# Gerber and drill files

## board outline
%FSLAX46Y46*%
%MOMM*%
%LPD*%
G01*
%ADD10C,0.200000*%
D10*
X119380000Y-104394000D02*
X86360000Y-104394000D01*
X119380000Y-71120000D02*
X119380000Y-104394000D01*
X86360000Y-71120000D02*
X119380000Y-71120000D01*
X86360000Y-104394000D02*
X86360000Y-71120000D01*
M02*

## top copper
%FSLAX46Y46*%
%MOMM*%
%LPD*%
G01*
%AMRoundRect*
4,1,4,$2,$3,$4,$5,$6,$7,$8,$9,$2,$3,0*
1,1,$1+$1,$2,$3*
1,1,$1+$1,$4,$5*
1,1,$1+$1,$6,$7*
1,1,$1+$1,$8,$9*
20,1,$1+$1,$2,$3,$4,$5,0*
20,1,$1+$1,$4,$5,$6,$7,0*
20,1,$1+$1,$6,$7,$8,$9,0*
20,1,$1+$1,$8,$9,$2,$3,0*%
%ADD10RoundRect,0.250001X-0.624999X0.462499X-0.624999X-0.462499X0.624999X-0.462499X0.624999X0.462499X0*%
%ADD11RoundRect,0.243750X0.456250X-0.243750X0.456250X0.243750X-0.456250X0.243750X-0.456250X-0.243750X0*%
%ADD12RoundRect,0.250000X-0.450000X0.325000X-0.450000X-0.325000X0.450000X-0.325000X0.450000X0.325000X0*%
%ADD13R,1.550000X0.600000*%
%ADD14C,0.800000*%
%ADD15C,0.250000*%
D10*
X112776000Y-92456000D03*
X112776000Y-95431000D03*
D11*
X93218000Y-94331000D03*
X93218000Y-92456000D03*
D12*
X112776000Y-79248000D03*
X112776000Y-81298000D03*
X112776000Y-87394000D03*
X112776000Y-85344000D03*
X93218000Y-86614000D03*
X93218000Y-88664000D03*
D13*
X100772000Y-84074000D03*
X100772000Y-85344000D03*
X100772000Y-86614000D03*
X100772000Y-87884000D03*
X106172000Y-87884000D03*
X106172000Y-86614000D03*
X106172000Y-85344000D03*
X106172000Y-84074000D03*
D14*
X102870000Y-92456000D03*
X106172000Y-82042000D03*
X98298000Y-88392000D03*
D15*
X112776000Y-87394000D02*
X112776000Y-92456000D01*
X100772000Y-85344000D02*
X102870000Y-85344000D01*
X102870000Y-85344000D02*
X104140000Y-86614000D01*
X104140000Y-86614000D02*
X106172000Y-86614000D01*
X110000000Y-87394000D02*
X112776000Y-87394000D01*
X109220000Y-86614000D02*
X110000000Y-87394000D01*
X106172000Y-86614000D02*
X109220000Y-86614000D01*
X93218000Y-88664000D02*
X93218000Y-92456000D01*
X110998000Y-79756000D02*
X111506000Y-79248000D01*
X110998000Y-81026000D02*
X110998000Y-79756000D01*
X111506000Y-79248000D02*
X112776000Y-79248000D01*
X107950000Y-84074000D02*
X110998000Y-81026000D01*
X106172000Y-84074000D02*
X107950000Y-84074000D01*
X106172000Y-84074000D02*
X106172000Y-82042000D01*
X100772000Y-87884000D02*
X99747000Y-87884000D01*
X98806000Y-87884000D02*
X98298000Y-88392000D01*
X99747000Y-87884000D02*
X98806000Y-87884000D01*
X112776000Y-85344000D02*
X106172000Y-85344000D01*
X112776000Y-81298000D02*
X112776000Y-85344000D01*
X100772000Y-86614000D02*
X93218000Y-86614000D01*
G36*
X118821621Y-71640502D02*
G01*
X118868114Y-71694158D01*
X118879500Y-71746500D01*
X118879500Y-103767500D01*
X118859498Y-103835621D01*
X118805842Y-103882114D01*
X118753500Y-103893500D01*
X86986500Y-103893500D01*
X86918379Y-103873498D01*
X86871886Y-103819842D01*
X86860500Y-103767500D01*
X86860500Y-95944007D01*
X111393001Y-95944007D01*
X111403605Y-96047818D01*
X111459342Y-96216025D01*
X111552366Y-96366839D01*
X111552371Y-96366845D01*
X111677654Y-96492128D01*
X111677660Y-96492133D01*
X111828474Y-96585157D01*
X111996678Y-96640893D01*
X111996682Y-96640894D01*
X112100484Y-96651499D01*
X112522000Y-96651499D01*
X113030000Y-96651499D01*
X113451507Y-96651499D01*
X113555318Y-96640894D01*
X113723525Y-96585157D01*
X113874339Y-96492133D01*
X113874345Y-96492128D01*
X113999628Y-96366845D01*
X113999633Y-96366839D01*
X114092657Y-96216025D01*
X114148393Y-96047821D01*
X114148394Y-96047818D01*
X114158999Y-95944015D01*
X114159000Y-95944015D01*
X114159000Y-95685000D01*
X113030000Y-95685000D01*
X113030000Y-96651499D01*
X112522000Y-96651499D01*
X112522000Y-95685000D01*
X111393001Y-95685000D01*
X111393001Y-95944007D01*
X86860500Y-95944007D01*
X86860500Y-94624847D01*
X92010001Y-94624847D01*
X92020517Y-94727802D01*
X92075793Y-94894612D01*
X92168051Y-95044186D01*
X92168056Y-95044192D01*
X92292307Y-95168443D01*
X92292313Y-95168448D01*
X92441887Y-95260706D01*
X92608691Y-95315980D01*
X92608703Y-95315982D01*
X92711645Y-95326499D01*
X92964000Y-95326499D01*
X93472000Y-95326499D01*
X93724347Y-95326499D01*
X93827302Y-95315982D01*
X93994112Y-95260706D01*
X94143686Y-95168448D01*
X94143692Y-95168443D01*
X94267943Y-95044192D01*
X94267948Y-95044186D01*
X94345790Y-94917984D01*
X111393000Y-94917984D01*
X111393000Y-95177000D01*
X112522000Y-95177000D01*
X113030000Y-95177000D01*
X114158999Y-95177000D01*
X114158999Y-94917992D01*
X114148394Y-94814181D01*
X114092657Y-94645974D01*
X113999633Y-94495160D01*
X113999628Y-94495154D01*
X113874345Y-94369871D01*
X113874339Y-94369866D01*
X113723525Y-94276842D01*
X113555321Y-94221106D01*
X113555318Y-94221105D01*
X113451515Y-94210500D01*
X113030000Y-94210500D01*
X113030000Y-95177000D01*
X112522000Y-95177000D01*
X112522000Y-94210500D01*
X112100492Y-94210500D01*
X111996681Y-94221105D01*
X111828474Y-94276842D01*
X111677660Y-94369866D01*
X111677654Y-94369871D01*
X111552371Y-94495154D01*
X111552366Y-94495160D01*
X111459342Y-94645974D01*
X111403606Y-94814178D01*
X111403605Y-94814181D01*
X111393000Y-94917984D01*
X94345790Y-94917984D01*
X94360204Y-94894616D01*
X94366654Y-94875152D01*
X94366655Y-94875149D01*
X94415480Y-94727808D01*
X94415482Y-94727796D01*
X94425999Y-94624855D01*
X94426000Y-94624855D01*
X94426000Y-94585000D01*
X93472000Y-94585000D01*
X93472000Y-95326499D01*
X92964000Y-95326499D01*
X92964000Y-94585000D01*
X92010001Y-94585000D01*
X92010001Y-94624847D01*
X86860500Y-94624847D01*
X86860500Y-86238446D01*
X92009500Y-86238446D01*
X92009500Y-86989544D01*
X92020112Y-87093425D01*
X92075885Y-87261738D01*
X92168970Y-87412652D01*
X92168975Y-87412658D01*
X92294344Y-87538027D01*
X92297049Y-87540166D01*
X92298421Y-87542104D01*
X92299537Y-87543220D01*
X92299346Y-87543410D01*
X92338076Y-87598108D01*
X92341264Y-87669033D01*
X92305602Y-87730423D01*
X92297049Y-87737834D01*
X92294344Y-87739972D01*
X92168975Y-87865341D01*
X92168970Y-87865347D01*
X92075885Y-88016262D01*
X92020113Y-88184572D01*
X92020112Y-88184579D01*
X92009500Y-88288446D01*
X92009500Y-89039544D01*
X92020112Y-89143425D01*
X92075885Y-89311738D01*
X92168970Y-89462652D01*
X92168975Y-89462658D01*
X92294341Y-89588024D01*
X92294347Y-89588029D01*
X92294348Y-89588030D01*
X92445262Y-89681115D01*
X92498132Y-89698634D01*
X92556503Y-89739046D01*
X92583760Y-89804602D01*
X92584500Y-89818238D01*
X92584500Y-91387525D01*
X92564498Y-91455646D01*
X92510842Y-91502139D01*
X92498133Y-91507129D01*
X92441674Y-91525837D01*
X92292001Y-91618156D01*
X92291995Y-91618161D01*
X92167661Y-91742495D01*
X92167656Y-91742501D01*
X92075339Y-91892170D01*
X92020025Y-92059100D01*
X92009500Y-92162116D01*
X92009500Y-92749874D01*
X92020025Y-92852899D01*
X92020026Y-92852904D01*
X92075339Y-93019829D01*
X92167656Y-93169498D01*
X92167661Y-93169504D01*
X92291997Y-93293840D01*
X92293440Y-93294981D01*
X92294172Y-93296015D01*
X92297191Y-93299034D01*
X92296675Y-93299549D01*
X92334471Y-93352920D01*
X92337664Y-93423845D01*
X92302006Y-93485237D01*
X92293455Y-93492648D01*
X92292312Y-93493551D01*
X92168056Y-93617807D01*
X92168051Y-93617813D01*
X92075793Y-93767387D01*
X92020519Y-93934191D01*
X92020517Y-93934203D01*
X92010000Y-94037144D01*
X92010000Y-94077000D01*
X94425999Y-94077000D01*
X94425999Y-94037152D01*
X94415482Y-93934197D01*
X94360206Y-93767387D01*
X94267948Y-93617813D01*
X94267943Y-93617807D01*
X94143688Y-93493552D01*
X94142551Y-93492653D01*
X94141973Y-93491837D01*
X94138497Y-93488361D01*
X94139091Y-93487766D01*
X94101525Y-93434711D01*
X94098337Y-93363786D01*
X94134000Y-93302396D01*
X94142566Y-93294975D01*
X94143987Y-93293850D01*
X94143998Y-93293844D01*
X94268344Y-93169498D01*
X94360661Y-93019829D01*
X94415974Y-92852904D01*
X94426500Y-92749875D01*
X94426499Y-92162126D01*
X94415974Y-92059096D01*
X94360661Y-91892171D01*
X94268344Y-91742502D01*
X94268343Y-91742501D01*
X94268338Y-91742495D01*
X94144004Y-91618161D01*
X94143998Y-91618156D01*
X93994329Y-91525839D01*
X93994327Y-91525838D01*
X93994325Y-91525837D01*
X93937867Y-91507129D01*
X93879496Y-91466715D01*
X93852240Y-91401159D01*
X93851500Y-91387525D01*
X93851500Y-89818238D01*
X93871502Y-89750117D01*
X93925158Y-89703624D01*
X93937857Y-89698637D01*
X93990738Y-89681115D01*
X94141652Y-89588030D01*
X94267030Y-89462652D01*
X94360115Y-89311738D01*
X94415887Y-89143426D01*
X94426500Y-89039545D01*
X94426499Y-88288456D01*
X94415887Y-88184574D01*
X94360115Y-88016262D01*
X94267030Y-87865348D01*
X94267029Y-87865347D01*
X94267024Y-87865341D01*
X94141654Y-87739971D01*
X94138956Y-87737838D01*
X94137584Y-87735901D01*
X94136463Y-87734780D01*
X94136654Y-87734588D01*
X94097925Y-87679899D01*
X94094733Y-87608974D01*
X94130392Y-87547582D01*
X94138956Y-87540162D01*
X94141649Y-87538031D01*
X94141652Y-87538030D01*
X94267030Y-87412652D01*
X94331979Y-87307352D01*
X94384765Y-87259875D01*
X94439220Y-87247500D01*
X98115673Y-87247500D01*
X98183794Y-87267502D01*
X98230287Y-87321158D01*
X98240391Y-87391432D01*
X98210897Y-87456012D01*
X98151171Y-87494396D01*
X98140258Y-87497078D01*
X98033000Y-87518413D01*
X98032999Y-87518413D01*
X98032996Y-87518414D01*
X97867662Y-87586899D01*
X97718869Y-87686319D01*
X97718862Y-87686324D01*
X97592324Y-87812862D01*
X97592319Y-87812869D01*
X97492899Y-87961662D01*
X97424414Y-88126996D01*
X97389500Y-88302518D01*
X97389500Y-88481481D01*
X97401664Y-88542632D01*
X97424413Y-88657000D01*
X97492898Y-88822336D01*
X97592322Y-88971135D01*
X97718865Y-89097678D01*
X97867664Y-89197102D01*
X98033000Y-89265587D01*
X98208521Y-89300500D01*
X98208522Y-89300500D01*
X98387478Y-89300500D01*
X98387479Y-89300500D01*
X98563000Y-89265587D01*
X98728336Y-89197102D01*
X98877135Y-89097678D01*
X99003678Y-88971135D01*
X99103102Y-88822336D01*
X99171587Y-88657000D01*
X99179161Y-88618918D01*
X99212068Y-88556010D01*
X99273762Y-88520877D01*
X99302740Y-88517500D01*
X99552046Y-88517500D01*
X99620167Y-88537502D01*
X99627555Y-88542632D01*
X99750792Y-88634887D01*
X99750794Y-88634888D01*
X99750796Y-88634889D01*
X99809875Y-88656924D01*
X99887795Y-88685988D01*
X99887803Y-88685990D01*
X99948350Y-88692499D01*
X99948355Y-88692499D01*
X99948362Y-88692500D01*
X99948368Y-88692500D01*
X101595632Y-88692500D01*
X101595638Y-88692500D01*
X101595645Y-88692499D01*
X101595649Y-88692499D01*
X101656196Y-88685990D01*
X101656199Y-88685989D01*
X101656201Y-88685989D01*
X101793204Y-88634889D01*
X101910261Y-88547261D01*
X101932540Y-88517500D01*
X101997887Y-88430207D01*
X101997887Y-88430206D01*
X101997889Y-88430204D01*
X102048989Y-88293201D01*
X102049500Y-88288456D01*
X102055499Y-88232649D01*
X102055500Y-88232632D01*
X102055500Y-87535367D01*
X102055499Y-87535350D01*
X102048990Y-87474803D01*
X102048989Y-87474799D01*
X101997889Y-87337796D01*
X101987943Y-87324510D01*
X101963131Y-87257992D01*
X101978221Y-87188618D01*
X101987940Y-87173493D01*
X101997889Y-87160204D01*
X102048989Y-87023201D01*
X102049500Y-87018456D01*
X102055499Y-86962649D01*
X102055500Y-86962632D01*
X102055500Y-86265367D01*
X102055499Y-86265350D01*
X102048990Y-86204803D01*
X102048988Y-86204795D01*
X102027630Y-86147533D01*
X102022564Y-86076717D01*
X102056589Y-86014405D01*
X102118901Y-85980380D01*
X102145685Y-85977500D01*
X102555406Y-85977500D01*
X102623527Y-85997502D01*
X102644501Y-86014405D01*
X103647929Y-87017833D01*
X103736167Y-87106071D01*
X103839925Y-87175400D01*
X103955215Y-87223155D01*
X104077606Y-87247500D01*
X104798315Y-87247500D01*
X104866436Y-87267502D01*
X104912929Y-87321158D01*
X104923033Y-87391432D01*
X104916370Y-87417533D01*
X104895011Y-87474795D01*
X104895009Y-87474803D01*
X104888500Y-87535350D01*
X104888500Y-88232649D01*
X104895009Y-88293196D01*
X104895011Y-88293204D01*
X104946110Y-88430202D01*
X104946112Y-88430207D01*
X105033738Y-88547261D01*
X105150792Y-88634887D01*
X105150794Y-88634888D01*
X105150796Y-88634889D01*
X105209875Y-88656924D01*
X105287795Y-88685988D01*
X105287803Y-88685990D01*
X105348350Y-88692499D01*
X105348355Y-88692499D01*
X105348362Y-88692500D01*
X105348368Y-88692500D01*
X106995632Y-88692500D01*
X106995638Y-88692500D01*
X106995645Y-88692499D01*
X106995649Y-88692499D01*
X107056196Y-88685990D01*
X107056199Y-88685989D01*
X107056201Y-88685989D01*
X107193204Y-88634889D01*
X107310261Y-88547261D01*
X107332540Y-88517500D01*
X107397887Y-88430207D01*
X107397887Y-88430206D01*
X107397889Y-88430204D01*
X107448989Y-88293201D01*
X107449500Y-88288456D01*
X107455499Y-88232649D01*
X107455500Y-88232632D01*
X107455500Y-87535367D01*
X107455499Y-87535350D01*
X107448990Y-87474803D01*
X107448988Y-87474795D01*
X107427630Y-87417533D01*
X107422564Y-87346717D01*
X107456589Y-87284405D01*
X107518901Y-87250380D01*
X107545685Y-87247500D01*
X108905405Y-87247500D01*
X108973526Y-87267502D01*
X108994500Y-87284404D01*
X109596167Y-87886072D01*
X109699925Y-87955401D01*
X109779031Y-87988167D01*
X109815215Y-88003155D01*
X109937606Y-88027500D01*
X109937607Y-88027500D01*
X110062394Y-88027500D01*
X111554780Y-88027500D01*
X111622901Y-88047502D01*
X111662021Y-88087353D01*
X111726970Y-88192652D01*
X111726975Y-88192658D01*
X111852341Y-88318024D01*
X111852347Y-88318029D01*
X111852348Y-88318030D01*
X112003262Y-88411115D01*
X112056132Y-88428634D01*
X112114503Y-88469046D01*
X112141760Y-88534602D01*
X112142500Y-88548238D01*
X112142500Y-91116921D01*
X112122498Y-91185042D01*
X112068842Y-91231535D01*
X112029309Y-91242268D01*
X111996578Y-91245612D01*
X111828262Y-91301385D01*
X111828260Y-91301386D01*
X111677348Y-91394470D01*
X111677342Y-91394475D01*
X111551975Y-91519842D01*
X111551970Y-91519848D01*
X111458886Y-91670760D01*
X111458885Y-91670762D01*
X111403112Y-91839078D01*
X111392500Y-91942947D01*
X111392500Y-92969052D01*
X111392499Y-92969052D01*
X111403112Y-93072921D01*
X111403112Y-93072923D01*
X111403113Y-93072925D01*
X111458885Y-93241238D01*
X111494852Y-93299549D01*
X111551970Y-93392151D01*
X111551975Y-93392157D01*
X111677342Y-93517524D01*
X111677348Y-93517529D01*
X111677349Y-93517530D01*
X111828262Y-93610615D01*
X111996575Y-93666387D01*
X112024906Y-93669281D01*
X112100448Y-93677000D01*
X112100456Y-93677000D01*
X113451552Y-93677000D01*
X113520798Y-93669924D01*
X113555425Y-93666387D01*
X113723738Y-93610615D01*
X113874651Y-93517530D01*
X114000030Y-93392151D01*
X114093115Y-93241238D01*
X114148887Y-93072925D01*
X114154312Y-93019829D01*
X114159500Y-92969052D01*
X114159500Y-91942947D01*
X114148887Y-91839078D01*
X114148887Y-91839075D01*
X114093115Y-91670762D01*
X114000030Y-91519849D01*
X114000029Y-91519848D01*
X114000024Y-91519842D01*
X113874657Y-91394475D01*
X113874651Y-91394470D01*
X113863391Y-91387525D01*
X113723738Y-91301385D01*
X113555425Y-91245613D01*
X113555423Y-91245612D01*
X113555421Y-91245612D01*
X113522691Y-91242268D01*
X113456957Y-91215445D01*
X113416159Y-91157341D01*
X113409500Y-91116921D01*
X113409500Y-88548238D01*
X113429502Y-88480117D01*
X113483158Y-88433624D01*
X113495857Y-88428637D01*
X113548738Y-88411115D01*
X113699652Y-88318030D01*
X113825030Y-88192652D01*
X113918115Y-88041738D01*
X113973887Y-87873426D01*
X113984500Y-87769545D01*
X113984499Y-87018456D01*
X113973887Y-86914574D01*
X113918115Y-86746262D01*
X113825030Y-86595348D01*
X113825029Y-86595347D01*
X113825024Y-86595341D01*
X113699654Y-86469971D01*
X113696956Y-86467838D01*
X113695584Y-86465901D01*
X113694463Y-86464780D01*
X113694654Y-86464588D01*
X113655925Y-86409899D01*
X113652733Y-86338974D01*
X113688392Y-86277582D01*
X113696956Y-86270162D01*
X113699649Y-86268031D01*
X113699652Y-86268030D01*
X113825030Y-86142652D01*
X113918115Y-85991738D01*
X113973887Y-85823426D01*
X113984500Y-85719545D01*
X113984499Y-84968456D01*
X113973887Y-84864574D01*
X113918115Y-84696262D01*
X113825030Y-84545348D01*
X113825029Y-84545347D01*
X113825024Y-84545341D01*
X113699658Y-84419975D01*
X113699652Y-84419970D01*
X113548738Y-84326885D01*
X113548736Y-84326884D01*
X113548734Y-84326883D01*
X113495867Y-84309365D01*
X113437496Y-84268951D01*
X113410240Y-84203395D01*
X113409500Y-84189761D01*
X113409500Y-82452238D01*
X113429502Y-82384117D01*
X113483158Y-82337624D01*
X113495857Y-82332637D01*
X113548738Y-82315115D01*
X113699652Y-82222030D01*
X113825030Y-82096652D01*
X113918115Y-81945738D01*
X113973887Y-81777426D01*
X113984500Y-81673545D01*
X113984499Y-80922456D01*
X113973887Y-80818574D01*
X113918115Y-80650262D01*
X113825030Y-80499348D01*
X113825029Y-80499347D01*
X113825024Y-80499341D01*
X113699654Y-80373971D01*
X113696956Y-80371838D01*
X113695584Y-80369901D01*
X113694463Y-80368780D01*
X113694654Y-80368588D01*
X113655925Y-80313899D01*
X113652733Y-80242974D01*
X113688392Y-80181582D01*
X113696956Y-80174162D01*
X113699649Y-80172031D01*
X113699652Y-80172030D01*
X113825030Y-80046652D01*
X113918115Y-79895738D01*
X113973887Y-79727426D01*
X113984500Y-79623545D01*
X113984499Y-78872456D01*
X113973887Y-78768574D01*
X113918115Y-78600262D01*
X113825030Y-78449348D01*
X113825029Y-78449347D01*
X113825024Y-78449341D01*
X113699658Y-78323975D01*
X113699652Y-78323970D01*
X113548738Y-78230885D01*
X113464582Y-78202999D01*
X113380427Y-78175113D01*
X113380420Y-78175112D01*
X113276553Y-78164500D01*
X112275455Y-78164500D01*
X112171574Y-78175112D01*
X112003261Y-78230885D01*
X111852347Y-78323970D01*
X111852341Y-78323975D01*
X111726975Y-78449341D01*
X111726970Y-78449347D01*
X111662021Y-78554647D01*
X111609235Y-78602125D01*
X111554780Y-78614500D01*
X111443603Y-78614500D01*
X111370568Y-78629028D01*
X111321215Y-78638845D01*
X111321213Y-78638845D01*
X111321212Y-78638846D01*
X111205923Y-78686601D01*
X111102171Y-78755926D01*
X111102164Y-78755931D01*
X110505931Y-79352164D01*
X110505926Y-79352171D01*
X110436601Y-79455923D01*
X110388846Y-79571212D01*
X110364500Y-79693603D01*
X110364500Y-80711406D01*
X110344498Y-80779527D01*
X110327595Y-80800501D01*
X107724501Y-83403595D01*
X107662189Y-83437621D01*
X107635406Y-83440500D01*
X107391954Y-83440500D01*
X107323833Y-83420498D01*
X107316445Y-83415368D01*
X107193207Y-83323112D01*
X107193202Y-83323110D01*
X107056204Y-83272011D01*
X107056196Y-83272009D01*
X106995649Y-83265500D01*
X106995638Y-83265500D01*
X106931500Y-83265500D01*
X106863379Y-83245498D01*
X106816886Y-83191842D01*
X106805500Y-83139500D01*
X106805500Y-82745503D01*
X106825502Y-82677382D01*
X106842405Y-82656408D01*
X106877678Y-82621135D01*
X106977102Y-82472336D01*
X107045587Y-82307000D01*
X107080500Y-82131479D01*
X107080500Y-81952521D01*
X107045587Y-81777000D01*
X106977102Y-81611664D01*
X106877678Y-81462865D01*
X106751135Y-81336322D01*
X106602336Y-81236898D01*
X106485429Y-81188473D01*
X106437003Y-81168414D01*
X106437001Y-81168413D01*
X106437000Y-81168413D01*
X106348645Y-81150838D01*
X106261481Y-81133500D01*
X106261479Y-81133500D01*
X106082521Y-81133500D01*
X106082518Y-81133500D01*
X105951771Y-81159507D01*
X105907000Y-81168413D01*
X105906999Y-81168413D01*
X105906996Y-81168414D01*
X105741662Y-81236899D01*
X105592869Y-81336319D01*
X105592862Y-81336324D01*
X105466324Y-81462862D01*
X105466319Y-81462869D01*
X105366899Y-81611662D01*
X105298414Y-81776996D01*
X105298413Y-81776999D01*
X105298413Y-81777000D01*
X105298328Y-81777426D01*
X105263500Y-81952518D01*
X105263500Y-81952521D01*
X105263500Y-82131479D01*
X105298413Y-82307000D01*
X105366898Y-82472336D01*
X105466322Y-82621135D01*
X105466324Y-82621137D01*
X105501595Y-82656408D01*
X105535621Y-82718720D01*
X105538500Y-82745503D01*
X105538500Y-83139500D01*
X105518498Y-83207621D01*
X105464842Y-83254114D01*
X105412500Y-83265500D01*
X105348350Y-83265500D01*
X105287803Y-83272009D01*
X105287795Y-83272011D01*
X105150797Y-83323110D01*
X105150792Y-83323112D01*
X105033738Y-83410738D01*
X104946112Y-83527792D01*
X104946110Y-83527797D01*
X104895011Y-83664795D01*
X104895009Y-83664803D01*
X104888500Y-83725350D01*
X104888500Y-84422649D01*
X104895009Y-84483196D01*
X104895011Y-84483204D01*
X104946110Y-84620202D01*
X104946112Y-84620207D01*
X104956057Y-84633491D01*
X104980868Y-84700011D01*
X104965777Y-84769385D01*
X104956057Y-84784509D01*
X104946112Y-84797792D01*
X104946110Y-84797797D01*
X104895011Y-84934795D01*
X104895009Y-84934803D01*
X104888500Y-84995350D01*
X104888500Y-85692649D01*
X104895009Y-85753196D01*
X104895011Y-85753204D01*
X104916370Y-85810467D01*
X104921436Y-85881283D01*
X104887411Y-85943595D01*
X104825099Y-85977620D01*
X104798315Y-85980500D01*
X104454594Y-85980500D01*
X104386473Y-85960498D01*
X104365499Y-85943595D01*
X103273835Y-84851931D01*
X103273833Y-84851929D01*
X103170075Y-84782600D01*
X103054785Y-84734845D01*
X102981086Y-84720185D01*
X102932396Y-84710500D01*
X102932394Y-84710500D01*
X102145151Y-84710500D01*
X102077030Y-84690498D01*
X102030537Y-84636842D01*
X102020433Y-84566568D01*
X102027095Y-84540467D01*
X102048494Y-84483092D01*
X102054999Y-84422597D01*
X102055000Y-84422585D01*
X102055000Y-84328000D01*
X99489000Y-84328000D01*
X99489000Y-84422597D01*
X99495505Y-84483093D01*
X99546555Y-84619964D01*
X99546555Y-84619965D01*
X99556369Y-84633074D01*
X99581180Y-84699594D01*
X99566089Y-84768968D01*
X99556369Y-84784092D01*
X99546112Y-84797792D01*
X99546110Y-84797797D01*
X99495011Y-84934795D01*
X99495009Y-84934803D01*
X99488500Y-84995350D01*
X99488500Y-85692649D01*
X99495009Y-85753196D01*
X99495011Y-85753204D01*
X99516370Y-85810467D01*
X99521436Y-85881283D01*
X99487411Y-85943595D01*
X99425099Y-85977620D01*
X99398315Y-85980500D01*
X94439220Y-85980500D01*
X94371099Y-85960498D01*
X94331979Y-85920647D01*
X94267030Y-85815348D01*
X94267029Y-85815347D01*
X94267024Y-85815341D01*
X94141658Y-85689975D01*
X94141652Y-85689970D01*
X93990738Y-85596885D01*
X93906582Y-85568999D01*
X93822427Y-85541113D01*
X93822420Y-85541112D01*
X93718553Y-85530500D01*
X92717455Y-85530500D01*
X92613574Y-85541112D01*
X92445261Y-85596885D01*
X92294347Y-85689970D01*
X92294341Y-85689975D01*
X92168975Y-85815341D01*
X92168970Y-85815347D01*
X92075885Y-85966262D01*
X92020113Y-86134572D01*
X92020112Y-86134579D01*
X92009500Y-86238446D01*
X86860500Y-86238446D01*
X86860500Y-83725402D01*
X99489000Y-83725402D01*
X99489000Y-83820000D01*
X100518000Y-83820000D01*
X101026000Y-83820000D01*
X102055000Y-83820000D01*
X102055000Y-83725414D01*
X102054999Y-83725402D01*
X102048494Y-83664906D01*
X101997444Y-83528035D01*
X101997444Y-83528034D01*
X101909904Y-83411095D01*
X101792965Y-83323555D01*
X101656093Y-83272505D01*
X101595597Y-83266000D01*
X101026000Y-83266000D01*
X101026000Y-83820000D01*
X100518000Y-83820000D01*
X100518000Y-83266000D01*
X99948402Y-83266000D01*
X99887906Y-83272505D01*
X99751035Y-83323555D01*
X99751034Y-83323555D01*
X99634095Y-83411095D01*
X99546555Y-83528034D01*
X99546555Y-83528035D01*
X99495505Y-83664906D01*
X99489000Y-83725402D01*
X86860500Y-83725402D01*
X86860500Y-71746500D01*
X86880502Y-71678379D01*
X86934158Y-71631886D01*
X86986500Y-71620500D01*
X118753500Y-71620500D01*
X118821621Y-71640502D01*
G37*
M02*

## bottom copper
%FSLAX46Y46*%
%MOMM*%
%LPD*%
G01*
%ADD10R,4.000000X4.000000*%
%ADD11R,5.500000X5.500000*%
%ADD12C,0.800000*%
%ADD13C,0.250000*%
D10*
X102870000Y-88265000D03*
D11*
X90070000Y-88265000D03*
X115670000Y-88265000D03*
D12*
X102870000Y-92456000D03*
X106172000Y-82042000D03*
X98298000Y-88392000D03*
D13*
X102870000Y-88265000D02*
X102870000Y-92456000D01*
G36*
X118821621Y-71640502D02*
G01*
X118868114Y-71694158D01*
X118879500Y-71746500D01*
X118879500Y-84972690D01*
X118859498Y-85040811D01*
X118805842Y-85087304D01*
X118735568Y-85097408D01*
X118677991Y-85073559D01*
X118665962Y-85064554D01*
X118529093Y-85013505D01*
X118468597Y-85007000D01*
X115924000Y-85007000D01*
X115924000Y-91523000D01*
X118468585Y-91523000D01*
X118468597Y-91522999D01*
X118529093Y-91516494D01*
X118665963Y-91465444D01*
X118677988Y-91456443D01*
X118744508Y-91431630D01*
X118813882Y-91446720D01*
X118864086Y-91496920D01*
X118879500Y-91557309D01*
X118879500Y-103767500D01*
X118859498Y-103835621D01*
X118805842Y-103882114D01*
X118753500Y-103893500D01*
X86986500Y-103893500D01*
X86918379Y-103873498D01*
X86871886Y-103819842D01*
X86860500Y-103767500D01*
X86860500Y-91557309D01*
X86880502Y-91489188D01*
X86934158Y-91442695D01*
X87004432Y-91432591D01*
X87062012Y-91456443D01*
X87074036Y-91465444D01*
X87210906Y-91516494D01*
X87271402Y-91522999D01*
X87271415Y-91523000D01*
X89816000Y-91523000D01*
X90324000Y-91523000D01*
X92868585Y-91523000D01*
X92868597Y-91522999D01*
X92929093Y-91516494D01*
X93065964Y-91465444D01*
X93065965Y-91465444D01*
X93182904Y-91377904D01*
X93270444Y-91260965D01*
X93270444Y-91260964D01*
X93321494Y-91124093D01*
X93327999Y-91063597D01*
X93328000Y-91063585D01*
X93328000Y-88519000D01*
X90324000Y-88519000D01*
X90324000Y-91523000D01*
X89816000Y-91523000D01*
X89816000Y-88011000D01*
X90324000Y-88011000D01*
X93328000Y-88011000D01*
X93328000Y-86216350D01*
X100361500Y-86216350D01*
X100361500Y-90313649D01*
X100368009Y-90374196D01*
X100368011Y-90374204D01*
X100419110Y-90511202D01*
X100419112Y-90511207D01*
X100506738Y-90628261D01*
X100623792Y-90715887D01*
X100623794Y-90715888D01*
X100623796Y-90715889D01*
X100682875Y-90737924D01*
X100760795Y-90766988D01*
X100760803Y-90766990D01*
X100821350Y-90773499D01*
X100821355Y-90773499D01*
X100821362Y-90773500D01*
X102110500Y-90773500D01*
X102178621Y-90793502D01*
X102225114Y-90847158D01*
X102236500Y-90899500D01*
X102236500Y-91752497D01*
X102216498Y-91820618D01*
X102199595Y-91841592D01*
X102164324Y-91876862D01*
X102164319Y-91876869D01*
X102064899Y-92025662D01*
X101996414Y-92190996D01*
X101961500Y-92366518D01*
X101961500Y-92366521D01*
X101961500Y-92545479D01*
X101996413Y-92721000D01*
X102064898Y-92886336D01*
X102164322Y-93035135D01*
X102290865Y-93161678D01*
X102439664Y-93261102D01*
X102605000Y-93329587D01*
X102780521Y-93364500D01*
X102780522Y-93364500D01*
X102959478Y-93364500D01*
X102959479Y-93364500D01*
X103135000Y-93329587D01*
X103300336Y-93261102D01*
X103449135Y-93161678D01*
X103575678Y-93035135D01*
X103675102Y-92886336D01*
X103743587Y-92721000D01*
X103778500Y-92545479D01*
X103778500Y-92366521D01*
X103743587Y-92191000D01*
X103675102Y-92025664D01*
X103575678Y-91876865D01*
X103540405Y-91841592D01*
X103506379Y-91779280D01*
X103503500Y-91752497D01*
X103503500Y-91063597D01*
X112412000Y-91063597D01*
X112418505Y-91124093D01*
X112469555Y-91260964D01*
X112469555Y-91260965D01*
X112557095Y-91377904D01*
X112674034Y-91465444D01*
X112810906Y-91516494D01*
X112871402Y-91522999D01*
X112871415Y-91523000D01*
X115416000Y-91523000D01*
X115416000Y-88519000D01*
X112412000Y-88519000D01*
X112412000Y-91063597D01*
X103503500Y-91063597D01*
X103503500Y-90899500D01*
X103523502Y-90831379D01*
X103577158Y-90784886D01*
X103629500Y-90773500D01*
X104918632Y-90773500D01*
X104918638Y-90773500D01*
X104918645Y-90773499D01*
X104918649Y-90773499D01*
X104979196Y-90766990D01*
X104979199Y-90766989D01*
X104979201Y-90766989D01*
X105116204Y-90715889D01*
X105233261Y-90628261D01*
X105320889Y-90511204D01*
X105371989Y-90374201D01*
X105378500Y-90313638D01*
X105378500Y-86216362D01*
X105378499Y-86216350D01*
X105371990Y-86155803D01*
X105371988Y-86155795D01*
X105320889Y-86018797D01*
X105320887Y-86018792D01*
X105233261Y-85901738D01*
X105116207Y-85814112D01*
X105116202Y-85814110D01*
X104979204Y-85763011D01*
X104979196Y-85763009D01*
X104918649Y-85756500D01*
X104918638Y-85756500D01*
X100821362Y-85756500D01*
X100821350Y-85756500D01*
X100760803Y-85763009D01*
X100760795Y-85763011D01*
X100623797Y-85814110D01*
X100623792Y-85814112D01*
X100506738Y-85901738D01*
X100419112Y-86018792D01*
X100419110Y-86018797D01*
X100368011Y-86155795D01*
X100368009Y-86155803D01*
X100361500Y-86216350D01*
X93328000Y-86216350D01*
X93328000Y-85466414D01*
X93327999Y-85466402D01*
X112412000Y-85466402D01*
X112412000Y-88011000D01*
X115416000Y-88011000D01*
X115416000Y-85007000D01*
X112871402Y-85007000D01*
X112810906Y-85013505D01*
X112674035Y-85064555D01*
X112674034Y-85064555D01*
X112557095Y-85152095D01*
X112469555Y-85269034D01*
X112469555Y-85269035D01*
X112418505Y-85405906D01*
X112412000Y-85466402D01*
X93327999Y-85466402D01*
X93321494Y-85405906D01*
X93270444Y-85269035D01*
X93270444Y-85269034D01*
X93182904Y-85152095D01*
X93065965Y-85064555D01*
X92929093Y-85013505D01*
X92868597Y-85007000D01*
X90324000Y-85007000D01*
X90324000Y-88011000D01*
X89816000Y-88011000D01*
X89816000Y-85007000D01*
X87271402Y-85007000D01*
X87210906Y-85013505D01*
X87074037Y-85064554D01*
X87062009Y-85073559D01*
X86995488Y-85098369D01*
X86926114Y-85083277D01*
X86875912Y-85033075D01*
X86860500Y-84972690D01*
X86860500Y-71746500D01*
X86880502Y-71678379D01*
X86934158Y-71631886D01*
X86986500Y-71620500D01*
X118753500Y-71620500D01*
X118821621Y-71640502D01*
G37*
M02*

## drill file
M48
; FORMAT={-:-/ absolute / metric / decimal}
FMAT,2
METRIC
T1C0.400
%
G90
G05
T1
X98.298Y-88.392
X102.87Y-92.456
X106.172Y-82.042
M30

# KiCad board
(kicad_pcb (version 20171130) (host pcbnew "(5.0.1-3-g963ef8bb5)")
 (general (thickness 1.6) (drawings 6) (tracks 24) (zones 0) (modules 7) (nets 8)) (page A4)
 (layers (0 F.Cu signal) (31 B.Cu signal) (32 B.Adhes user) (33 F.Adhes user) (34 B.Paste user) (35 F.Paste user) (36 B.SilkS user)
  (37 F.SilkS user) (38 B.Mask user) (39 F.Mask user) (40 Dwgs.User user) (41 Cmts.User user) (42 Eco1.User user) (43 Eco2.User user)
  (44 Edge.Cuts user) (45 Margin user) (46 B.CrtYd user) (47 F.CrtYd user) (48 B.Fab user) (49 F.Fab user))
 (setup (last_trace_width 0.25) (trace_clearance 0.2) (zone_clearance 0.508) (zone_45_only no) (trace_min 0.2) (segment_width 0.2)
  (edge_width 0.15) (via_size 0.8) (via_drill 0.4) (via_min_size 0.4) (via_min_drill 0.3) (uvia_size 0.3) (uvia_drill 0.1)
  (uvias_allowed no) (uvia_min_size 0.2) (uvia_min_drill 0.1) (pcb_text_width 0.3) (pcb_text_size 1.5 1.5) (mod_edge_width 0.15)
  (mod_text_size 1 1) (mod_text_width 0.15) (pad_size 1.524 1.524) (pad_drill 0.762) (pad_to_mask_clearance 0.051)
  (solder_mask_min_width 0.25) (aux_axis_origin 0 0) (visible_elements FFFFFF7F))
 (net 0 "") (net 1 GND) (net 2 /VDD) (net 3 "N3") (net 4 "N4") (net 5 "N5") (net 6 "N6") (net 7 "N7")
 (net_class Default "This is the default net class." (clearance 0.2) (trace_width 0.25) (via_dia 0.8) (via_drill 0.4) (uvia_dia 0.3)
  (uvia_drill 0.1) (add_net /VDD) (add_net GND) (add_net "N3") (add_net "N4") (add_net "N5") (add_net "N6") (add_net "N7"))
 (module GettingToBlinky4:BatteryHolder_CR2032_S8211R (layer B.Cu) (at 102.87 88.265)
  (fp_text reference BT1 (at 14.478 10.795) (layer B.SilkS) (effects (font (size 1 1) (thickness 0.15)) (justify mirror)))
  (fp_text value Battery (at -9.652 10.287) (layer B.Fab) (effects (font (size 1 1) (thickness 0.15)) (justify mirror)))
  (pad 2 smd rect (at 0 0) (size 4 4) (layers B.Cu B.Paste B.Mask) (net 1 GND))
  (pad 1 smd rect (at -12.8 0) (size 5.5 5.5) (layers B.Cu B.Paste B.Mask) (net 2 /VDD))
  (pad 1 smd rect (at 12.8 0) (size 5.5 5.5) (layers B.Cu B.Paste B.Mask) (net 2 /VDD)))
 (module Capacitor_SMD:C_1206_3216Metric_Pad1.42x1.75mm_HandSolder (layer F.Cu) (at 112.776 93.9435 270)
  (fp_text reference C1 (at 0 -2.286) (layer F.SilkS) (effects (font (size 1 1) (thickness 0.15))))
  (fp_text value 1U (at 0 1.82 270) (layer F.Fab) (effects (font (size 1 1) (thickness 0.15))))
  (pad 1 smd roundrect (at -1.4875 0 270) (size 1.425 1.75) (layers F.Cu F.Paste F.Mask) (roundrect_rratio 0.175439) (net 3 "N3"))
  (pad 2 smd roundrect (at 1.4875 0 270) (size 1.425 1.75) (layers F.Cu F.Paste F.Mask) (roundrect_rratio 0.175439) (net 1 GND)))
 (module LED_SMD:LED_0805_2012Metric (layer F.Cu) (at 93.218 93.3935 90)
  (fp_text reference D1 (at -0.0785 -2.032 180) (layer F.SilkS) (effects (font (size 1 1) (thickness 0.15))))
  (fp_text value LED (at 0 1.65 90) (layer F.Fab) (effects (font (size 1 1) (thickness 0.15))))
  (pad 1 smd roundrect (at -0.9375 0 90) (size 0.975 1.4) (layers F.Cu F.Paste F.Mask) (roundrect_rratio 0.25) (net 1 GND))
  (pad 2 smd roundrect (at 0.9375 0 90) (size 0.975 1.4) (layers F.Cu F.Paste F.Mask) (roundrect_rratio 0.25) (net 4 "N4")))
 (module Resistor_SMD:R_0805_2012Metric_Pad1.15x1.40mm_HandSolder (layer F.Cu) (at 112.776 80.273 270)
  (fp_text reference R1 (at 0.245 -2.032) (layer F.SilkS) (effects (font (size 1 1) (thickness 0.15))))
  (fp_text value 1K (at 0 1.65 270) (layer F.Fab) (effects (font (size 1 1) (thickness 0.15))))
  (pad 1 smd roundrect (at -1.025 0 270) (size 1.15 1.4) (layers F.Cu F.Paste F.Mask) (roundrect_rratio 0.217391) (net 2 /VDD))
  (pad 2 smd roundrect (at 1.025 0 270) (size 1.15 1.4) (layers F.Cu F.Paste F.Mask) (roundrect_rratio 0.217391) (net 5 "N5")))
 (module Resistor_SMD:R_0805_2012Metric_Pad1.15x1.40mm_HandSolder (layer F.Cu) (at 112.776 86.369 270)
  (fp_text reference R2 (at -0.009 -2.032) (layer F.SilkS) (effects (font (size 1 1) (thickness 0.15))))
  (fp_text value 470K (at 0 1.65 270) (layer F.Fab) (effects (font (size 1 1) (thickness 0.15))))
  (pad 2 smd roundrect (at 1.025 0 270) (size 1.15 1.4) (layers F.Cu F.Paste F.Mask) (roundrect_rratio 0.217391) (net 3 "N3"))
  (pad 1 smd roundrect (at -1.025 0 270) (size 1.15 1.4) (layers F.Cu F.Paste F.Mask) (roundrect_rratio 0.217391) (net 5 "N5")))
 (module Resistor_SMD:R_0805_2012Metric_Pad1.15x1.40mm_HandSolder (layer F.Cu) (at 93.218 87.639 270)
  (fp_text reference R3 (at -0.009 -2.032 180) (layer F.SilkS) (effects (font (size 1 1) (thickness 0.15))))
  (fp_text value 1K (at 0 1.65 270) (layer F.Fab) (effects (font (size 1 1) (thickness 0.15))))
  (pad 1 smd roundrect (at -1.025 0 270) (size 1.15 1.4) (layers F.Cu F.Paste F.Mask) (roundrect_rratio 0.217391) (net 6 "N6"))
  (pad 2 smd roundrect (at 1.025 0 270) (size 1.15 1.4) (layers F.Cu F.Paste F.Mask) (roundrect_rratio 0.217391) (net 4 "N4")))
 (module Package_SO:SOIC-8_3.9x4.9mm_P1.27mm (layer F.Cu) (at 103.472 85.979)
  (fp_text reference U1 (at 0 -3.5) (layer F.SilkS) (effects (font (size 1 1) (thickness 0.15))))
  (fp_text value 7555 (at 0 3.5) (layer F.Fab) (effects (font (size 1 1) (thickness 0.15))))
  (pad 1 smd rect (at -2.7 -1.905) (size 1.55 0.6) (layers F.Cu F.Paste F.Mask) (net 1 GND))
  (pad 2 smd rect (at -2.7 -0.635) (size 1.55 0.6) (layers F.Cu F.Paste F.Mask) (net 3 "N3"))
  (pad 3 smd rect (at -2.7 0.635) (size 1.55 0.6) (layers F.Cu F.Paste F.Mask) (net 6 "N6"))
  (pad 4 smd rect (at -2.7 1.905) (size 1.55 0.6) (layers F.Cu F.Paste F.Mask) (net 2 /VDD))
  (pad 5 smd rect (at 2.7 1.905) (size 1.55 0.6) (layers F.Cu F.Paste F.Mask) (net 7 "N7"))
  (pad 6 smd rect (at 2.7 0.635) (size 1.55 0.6) (layers F.Cu F.Paste F.Mask) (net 3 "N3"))
  (pad 7 smd rect (at 2.7 -0.635) (size 1.55 0.6) (layers F.Cu F.Paste F.Mask) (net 5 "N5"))
  (pad 8 smd rect (at 2.7 -1.905) (size 1.55 0.6) (layers F.Cu F.Paste F.Mask) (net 2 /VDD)))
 (gr_line (start 119.38 104.394) (end 86.36 104.394) (layer Edge.Cuts) (width 0.2))
 (gr_line (start 119.38 71.12) (end 119.38 104.394) (layer Edge.Cuts) (width 0.2))
 (gr_line (start 86.36 71.12) (end 119.38 71.12) (layer Edge.Cuts) (width 0.2))
 (gr_line (start 86.36 104.394) (end 86.36 71.12) (layer Edge.Cuts) (width 0.2))
 (segment (start 112.776 87.394) (end 112.776 92.456) (width 0.25) (layer F.Cu) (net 3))
 (segment (start 100.772 85.344) (end 102.87 85.344) (width 0.25) (layer F.Cu) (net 3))
 (segment (start 102.87 85.344) (end 104.14 86.614) (width 0.25) (layer F.Cu) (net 3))
 (segment (start 104.14 86.614) (end 106.172 86.614) (width 0.25) (layer F.Cu) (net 3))
 (segment (start 110 87.394) (end 112.776 87.394) (width 0.25) (layer F.Cu) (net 3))
 (segment (start 109.22 86.614) (end 110 87.394) (width 0.25) (layer F.Cu) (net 3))
 (segment (start 106.172 86.614) (end 109.22 86.614) (width 0.25) (layer F.Cu) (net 3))
 (via (at 102.87 92.456) (size 0.8) (drill 0.4) (layers F.Cu B.Cu) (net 1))
 (segment (start 102.87 88.265) (end 102.87 92.456) (width 0.25) (layer B.Cu) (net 1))
 (segment (start 93.218 88.664) (end 93.218 92.456) (width 0.25) (layer F.Cu) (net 4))
 (segment (start 110.998 79.756) (end 111.506 79.248) (width 0.25) (layer F.Cu) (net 2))
 (segment (start 110.998 81.026) (end 110.998 79.756) (width 0.25) (layer F.Cu) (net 2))
 (segment (start 111.506 79.248) (end 112.776 79.248) (width 0.25) (layer F.Cu) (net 2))
 (segment (start 107.95 84.074) (end 110.998 81.026) (width 0.25) (layer F.Cu) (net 2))
 (segment (start 106.172 84.074) (end 107.95 84.074) (width 0.25) (layer F.Cu) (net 2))
 (via (at 106.172 82.042) (size 0.8) (drill 0.4) (layers F.Cu B.Cu) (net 2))
 (segment (start 106.172 84.074) (end 106.172 82.042) (width 0.25) (layer F.Cu) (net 2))
 (segment (start 100.772 87.884) (end 99.747 87.884) (width 0.25) (layer F.Cu) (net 2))
 (via (at 98.298 88.392) (size 0.8) (drill 0.4) (layers F.Cu B.Cu) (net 2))
 (segment (start 98.806 87.884) (end 98.298 88.392) (width 0.25) (layer F.Cu) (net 2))
 (segment (start 99.747 87.884) (end 98.806 87.884) (width 0.25) (layer F.Cu) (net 2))
 (segment (start 112.776 85.344) (end 106.172 85.344) (width 0.25) (layer F.Cu) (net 5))
 (segment (start 112.776 81.298) (end 112.776 85.344) (width 0.25) (layer F.Cu) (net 5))
 (segment (start 100.772 86.614) (end 93.218 86.614) (width 0.25) (layer F.Cu) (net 6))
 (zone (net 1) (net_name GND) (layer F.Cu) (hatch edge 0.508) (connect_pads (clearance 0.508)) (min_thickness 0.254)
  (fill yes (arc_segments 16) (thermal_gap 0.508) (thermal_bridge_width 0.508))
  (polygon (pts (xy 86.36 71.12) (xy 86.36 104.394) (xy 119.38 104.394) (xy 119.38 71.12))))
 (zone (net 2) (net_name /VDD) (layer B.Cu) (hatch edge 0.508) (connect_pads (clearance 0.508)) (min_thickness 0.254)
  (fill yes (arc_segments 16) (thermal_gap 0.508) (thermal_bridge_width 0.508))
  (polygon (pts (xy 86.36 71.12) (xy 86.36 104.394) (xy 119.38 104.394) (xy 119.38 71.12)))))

